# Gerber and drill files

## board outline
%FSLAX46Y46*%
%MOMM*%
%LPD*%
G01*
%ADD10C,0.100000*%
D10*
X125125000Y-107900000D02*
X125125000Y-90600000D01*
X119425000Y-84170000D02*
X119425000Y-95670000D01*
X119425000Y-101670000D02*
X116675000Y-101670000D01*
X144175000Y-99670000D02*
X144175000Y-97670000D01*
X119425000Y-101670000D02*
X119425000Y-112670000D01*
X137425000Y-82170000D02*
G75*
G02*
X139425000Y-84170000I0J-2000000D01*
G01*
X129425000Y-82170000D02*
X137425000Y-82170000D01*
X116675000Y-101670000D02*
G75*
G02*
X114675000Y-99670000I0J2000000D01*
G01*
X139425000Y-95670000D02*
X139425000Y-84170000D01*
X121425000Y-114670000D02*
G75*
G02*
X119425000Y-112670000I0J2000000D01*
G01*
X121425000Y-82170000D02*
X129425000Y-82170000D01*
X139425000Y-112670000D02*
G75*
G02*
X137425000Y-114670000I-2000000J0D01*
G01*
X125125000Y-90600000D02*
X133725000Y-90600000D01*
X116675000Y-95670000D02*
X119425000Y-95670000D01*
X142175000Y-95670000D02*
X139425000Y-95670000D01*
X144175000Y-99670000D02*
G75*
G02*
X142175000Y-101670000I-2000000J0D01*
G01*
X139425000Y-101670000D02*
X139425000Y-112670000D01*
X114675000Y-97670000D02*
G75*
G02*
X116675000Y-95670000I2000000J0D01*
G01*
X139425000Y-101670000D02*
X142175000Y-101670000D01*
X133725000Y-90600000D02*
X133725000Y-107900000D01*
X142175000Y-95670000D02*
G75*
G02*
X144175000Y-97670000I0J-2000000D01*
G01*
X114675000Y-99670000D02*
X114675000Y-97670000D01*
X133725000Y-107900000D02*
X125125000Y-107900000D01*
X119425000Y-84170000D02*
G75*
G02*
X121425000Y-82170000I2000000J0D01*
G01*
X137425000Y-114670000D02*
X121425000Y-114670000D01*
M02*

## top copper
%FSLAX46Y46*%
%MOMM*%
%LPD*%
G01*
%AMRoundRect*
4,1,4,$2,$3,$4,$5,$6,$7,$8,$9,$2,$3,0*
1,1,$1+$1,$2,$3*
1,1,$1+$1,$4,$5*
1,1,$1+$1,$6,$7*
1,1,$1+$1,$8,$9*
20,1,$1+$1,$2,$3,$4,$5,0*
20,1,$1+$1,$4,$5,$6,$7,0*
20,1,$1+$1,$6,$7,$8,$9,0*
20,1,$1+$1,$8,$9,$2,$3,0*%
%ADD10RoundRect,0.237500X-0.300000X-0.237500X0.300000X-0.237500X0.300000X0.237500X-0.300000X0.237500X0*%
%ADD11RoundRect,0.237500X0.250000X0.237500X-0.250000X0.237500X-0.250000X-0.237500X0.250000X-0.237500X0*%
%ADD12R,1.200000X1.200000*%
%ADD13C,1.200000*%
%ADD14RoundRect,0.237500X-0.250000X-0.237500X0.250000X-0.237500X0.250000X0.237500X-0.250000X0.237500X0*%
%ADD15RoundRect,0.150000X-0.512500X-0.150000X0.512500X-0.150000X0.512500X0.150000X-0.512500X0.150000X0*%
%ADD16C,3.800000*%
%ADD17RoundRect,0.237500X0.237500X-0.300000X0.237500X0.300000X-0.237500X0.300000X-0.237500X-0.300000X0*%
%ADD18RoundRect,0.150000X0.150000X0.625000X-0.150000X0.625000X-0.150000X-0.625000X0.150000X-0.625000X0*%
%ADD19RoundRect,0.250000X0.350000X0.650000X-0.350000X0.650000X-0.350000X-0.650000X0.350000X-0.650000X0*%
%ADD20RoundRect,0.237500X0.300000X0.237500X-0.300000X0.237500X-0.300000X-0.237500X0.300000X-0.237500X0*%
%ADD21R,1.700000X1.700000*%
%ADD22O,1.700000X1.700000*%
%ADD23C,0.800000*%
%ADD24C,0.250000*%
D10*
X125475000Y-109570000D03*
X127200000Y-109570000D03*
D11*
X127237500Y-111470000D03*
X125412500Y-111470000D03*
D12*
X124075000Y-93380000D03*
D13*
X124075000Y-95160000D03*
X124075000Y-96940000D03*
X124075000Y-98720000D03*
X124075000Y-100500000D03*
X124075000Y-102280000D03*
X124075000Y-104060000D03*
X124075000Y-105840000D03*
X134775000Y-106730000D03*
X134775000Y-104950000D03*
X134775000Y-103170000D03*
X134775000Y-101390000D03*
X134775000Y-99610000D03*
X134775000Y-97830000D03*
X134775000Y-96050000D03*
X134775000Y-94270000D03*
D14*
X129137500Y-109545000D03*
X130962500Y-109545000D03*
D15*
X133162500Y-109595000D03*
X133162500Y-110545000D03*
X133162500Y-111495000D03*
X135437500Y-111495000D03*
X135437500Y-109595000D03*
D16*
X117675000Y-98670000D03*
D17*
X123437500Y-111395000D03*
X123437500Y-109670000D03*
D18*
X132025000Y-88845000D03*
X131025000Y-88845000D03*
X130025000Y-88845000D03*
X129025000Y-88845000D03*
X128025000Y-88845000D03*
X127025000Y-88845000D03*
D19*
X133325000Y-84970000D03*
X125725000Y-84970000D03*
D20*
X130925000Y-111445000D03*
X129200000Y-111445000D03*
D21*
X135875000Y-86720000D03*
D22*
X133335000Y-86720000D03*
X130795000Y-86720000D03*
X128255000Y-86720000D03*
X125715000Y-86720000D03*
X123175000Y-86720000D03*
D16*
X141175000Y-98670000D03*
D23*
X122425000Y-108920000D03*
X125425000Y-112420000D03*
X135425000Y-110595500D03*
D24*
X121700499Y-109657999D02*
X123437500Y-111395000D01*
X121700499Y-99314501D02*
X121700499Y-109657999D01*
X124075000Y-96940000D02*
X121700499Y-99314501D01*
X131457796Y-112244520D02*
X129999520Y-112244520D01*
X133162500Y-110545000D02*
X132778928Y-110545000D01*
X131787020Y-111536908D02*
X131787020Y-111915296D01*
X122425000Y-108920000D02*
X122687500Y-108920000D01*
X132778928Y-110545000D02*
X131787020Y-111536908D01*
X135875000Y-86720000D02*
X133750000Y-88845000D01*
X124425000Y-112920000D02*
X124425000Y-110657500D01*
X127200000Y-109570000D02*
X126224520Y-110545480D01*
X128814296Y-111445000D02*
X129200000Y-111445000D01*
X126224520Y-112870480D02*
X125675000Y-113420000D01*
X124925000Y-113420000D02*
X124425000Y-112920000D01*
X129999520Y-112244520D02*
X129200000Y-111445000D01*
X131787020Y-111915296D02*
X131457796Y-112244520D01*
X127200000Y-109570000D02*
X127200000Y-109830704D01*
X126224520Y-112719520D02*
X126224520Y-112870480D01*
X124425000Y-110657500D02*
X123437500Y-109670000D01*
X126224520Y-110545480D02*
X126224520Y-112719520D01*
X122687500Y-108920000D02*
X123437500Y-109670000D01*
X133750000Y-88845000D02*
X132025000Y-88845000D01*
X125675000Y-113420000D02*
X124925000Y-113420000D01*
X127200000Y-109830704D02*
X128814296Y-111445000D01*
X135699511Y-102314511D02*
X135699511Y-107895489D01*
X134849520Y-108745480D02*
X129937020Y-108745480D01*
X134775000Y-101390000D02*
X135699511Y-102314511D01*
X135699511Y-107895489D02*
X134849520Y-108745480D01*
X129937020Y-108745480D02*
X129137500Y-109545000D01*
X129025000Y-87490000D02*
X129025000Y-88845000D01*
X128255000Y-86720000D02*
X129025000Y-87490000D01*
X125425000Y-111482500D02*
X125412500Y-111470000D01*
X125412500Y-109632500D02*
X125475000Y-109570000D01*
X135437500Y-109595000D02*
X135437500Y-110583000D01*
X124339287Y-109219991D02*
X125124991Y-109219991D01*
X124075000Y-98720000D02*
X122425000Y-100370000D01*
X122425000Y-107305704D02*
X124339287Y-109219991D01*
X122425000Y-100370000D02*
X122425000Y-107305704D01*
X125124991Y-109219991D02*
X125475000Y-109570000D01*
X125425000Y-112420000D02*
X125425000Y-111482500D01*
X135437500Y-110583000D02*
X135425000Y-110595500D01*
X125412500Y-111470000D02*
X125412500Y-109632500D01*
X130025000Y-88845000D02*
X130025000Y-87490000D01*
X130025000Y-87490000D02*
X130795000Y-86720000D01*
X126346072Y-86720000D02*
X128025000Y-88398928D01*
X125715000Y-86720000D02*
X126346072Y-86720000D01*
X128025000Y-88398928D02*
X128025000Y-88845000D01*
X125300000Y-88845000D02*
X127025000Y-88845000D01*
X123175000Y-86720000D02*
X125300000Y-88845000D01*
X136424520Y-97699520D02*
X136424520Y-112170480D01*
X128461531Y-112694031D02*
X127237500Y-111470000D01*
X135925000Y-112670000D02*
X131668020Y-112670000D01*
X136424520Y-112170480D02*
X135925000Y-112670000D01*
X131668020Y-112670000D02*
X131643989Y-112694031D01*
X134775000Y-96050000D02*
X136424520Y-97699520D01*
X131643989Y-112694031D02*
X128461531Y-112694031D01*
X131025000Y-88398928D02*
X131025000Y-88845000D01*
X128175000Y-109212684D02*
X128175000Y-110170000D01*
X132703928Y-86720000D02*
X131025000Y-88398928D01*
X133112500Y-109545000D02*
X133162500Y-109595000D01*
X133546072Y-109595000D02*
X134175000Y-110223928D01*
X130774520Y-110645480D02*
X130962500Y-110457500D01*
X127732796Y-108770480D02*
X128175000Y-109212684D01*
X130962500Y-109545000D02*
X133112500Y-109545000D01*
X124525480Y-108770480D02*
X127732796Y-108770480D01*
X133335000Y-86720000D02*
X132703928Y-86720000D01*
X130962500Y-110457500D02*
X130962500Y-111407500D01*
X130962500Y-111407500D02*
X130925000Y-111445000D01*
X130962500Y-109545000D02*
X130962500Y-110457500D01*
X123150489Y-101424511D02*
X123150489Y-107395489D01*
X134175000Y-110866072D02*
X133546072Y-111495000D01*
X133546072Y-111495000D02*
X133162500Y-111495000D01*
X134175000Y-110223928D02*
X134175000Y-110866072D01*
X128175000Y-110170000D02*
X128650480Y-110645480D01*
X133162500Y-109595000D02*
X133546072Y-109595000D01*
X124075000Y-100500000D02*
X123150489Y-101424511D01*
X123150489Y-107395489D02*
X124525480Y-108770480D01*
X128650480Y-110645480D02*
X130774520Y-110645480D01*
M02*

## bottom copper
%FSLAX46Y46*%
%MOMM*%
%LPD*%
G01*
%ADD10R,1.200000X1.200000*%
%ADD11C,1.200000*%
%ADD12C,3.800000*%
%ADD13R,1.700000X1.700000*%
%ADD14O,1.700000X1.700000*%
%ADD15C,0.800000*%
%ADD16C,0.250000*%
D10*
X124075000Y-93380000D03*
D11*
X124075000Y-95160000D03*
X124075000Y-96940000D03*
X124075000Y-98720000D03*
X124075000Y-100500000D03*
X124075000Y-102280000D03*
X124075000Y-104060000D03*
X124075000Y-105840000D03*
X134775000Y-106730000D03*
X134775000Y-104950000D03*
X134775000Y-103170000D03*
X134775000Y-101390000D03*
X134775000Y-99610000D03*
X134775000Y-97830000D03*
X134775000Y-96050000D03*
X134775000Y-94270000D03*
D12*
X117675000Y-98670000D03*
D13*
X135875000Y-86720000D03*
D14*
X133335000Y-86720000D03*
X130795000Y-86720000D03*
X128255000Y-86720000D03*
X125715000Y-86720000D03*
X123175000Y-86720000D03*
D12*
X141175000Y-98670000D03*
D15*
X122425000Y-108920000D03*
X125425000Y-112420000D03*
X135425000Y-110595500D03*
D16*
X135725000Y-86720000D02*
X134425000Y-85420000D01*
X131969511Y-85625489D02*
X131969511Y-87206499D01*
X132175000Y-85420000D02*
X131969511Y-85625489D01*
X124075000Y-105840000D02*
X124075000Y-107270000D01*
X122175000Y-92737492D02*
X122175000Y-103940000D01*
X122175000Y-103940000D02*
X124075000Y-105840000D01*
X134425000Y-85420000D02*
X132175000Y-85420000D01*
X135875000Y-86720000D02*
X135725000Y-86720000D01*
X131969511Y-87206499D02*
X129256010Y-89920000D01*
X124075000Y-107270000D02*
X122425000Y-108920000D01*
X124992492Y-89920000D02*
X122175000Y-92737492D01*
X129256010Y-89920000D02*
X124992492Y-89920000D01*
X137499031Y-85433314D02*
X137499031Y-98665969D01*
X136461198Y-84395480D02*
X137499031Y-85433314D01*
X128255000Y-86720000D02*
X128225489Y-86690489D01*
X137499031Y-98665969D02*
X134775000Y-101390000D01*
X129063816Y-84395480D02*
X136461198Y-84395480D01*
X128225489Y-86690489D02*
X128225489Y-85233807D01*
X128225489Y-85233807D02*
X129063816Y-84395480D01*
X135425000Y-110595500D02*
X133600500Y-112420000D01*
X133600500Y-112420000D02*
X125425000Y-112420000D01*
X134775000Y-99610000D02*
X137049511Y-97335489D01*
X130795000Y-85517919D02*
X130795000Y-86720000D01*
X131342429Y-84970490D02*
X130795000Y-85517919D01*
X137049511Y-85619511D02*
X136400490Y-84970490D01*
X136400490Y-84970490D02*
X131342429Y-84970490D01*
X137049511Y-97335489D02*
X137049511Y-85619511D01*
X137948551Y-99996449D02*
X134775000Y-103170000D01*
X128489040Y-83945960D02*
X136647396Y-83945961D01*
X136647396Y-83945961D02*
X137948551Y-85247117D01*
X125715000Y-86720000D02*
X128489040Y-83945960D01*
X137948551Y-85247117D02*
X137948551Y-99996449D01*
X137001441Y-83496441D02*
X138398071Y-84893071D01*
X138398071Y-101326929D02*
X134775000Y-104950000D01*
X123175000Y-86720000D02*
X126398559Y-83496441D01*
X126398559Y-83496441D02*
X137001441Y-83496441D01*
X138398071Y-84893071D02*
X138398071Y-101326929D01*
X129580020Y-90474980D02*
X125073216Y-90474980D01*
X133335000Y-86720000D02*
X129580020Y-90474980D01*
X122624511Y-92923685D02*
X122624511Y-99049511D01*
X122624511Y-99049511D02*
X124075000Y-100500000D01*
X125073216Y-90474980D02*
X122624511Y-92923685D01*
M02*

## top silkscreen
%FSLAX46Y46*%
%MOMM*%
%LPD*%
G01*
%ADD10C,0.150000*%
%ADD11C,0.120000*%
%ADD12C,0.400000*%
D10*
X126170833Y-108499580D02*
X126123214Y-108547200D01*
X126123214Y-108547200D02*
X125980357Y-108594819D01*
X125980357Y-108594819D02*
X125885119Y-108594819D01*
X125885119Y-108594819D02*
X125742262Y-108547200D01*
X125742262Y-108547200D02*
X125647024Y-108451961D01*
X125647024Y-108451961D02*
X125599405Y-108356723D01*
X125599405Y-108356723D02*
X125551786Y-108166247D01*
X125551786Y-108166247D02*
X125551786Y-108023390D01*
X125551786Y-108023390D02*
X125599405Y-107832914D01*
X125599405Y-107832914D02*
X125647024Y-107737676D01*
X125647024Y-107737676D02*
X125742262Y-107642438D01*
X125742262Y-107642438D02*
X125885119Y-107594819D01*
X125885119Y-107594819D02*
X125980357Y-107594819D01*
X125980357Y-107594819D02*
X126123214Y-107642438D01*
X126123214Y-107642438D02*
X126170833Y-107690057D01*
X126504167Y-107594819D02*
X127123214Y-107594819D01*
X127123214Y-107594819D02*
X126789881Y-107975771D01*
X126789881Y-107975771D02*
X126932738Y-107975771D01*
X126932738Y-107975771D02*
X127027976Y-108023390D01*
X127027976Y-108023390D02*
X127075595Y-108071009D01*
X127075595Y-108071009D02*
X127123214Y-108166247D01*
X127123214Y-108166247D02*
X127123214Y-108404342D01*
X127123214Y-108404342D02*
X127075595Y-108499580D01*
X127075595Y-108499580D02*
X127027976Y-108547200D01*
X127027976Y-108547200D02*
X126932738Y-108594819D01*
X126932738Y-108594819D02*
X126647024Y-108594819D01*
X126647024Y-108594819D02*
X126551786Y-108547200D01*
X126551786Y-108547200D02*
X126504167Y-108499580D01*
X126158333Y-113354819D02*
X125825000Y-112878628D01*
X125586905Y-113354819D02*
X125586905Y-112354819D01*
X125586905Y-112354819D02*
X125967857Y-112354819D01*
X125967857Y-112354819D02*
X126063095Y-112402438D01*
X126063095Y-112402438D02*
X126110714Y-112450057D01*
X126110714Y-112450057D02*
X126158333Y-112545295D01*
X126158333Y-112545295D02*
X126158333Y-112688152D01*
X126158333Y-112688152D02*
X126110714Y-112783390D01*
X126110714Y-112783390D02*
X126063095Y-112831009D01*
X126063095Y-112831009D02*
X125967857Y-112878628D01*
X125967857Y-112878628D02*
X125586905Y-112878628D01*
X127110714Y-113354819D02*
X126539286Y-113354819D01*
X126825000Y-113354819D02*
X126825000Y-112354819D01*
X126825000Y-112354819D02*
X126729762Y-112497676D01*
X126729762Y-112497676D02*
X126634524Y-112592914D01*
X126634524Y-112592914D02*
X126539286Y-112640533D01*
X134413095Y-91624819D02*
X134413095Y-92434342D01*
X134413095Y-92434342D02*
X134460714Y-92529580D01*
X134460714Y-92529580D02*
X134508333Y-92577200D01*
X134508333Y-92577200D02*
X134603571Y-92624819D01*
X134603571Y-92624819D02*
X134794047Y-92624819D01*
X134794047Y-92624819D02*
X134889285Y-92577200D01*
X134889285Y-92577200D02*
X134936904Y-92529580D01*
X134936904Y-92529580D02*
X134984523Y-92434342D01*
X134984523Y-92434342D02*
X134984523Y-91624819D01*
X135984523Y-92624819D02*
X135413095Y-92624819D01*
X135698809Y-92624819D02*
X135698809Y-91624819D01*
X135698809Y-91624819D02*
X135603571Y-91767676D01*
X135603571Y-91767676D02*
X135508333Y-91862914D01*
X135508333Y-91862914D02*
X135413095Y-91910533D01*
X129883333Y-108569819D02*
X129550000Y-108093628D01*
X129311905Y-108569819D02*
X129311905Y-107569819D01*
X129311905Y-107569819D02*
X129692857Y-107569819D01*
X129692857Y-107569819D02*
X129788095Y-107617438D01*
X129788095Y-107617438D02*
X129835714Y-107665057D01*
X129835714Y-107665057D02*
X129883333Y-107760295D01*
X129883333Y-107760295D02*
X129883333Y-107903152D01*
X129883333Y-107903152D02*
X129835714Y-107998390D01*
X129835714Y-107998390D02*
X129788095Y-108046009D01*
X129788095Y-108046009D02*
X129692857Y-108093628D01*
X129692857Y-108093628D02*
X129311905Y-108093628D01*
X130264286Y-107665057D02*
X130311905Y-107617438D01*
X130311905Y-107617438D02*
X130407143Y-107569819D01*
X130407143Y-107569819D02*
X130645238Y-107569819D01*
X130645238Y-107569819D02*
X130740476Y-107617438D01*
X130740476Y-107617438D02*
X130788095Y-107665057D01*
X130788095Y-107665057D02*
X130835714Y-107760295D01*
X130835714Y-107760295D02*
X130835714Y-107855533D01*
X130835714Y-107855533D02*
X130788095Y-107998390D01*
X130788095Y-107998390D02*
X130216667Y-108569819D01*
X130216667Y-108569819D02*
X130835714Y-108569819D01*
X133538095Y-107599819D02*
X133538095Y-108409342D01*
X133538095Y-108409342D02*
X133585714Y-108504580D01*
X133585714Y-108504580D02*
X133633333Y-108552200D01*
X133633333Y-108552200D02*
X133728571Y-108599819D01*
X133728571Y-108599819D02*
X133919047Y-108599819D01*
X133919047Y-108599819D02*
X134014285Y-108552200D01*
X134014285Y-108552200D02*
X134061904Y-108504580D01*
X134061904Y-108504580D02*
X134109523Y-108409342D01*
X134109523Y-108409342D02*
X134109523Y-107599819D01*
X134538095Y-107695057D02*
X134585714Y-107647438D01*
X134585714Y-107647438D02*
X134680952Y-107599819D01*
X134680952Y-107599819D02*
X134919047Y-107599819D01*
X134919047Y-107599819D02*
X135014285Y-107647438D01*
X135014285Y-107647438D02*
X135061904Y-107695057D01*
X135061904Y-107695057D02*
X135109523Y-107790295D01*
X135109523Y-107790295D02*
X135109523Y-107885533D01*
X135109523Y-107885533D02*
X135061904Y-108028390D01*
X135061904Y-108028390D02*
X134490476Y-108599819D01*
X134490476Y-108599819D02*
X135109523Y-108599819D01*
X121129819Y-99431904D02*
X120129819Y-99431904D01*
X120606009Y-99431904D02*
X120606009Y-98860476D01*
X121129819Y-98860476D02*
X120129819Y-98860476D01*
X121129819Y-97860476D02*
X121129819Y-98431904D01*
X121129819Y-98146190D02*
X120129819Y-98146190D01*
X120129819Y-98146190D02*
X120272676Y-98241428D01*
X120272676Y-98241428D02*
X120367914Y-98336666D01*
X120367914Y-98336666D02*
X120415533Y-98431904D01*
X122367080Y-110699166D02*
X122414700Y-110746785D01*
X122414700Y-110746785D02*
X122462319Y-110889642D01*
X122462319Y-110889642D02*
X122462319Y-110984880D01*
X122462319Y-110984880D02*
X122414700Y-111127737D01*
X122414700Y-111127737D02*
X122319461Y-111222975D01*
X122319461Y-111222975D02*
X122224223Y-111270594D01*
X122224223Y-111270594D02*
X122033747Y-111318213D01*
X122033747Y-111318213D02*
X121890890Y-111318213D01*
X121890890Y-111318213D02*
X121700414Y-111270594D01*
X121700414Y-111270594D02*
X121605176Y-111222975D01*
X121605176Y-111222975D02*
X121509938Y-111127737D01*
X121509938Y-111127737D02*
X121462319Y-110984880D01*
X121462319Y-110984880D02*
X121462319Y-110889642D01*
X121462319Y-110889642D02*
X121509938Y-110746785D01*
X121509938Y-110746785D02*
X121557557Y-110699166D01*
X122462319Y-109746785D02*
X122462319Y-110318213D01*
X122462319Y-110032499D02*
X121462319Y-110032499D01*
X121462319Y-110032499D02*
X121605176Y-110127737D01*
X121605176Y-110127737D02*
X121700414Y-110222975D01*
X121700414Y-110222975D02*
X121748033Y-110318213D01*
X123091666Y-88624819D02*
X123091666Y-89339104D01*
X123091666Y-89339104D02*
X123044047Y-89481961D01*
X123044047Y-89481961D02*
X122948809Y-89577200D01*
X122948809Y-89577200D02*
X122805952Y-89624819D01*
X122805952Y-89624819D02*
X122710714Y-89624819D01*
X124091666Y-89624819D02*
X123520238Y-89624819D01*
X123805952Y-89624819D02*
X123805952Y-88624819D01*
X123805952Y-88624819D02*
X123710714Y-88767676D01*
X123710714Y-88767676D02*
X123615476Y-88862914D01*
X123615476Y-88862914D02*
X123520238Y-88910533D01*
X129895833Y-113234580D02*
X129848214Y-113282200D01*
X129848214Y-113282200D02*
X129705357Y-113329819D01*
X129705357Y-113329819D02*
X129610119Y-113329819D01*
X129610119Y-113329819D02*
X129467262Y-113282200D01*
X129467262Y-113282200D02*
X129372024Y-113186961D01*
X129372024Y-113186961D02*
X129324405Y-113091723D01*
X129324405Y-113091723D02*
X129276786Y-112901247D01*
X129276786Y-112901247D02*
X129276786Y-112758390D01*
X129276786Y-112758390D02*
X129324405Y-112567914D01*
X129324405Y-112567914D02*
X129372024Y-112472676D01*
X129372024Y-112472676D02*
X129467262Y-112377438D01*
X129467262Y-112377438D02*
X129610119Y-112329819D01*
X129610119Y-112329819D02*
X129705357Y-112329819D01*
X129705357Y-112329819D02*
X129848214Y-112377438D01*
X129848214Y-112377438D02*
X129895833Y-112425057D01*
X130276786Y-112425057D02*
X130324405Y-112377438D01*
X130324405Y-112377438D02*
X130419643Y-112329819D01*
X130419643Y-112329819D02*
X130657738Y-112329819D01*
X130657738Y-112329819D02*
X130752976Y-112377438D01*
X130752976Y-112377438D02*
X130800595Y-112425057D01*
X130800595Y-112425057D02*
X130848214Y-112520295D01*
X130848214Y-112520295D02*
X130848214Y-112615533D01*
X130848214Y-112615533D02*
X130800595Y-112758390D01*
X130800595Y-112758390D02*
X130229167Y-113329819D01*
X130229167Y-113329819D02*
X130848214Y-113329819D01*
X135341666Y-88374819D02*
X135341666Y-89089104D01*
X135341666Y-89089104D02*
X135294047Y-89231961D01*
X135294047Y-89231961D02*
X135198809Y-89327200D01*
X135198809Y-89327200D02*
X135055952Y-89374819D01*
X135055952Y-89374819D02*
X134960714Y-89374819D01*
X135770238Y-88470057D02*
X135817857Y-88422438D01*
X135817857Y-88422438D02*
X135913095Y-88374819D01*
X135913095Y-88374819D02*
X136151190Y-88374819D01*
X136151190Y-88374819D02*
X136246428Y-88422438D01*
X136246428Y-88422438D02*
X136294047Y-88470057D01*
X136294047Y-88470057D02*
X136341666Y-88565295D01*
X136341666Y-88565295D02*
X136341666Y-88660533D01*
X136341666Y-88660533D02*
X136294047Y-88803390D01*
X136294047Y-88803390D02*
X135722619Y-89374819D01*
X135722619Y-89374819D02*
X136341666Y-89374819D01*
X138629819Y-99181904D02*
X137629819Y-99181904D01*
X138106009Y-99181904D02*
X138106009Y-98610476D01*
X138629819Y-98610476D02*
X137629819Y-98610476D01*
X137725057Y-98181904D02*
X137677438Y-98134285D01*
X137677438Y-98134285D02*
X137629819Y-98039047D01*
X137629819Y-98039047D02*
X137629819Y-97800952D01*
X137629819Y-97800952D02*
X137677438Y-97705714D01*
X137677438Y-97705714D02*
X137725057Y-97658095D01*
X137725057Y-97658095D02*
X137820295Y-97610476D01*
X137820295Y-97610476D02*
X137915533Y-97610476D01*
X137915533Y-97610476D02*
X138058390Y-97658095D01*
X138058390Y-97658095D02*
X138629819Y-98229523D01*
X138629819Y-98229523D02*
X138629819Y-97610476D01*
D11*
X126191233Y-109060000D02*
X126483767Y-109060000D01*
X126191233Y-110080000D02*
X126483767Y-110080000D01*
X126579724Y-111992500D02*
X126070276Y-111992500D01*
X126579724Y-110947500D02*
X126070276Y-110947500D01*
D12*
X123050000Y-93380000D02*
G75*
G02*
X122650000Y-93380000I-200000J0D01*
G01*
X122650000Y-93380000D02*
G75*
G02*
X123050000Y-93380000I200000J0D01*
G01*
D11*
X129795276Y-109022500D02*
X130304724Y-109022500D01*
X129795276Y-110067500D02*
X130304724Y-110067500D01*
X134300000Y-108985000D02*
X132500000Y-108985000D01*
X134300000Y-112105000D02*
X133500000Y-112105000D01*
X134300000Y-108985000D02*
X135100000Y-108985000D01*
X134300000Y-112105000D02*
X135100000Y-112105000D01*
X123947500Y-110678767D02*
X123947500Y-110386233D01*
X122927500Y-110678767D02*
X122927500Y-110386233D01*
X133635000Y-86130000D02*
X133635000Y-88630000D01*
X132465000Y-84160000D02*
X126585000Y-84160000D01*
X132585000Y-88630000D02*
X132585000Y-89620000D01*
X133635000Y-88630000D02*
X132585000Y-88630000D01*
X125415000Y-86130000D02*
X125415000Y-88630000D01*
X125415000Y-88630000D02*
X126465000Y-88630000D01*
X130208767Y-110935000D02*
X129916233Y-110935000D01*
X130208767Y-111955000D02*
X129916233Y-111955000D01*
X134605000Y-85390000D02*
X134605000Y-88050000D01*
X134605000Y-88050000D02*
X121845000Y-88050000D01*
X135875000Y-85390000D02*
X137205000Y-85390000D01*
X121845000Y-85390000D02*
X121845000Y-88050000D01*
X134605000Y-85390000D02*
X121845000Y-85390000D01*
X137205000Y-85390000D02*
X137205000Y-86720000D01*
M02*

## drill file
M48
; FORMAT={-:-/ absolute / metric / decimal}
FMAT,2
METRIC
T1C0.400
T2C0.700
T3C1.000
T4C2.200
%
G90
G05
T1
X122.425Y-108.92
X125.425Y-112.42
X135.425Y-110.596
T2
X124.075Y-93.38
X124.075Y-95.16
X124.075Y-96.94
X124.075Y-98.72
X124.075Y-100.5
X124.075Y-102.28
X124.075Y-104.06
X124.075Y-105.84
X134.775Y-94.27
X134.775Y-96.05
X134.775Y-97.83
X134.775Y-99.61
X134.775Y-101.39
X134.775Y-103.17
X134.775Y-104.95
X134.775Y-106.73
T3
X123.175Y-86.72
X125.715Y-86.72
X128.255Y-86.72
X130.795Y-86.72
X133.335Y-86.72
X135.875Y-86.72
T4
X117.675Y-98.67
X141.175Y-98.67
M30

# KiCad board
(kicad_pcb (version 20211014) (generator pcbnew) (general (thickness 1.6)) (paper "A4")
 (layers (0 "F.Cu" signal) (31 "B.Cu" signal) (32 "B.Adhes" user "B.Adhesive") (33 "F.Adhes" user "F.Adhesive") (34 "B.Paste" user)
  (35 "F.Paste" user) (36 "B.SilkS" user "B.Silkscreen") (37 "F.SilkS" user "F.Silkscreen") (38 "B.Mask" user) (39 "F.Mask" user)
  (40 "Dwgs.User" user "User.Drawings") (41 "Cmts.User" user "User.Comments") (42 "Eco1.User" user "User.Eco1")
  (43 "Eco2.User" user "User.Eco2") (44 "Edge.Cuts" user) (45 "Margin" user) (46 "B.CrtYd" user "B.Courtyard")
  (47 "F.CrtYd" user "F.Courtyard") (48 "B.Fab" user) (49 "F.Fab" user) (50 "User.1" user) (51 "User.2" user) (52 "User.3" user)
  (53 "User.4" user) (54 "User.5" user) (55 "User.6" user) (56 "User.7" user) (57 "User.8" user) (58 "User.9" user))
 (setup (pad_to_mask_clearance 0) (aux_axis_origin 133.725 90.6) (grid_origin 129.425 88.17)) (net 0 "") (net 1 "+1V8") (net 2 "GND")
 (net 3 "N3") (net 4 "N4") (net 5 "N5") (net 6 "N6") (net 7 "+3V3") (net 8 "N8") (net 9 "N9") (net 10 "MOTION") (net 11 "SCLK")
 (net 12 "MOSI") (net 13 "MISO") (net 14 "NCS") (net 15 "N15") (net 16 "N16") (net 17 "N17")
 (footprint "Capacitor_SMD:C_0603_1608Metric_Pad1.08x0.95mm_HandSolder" (layer "F.Cu") (at 126.3375 109.57)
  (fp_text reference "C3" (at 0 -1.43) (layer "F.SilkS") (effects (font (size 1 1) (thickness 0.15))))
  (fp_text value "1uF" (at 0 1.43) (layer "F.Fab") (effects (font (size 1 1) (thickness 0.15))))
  (fp_line (start -0.146267 -0.51) (end 0.146267 -0.51) (layer "F.SilkS") (width 0.12))
  (fp_line (start -0.146267 0.51) (end 0.146267 0.51) (layer "F.SilkS") (width 0.12))
  (pad "1" smd roundrect (at -0.8625 0) (size 1.075 0.95) (layers "F.Cu" "F.Paste" "F.Mask") (roundrect_rratio 0.25) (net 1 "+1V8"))
  (pad "2" smd roundrect (at 0.8625 0) (size 1.075 0.95) (layers "F.Cu" "F.Paste" "F.Mask") (roundrect_rratio 0.25) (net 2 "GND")))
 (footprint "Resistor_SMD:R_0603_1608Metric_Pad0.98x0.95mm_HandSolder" (layer "F.Cu") (at 126.325 111.47 180)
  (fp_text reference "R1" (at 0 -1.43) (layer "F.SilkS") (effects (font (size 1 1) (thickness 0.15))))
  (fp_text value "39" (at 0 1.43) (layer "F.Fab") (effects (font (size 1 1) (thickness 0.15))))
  (fp_line (start -0.254724 -0.5225) (end 0.254724 -0.5225) (layer "F.SilkS") (width 0.12))
  (fp_line (start -0.254724 0.5225) (end 0.254724 0.5225) (layer "F.SilkS") (width 0.12))
  (pad "1" smd roundrect (at -0.9125 0 180) (size 0.975 0.95) (layers "F.Cu" "F.Paste" "F.Mask") (roundrect_rratio 0.25) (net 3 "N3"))
  (pad "2" smd roundrect (at 0.9125 0 180) (size 0.975 0.95) (layers "F.Cu" "F.Paste" "F.Mask") (roundrect_rratio 0.25) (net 1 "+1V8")))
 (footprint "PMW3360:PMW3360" (layer "F.Cu") (at 124.075 93.38)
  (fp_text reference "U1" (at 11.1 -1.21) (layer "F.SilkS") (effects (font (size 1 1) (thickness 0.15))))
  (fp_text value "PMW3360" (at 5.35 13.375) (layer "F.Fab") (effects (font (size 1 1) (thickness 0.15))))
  (fp_circle (center -1.225 0) (end -1.025 0) (layer "F.SilkS") (width 0.4) (fill none))
  (pad "1" thru_hole rect (at 0 0) (size 1.2 1.2) (drill 0.7) (layers *.Cu *.Mask) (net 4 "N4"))
  (pad "2" thru_hole circle (at 0 1.78) (size 1.2 1.2) (drill 0.7) (layers *.Cu *.Mask) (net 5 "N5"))
  (pad "3" thru_hole circle (at 0 3.56) (size 1.2 1.2) (drill 0.7) (layers *.Cu *.Mask) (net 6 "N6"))
  (pad "4" thru_hole circle (at 0 5.34) (size 1.2 1.2) (drill 0.7) (layers *.Cu *.Mask) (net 1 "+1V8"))
  (pad "5" thru_hole circle (at 0 7.12) (size 1.2 1.2) (drill 0.7) (layers *.Cu *.Mask) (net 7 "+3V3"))
  (pad "6" thru_hole circle (at 0 8.9) (size 1.2 1.2) (drill 0.7) (layers *.Cu *.Mask) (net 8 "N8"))
  (pad "7" thru_hole circle (at 0 10.68) (size 1.2 1.2) (drill 0.7) (layers *.Cu *.Mask) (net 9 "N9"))
  (pad "8" thru_hole circle (at 0 12.46) (size 1.2 1.2) (drill 0.7) (layers *.Cu *.Mask) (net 2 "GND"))
  (pad "9" thru_hole circle (at 10.7 13.35) (size 1.2 1.2) (drill 0.7) (layers *.Cu *.Mask) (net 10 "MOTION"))
  (pad "10" thru_hole circle (at 10.7 11.57) (size 1.2 1.2) (drill 0.7) (layers *.Cu *.Mask) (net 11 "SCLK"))
  (pad "11" thru_hole circle (at 10.7 9.79) (size 1.2 1.2) (drill 0.7) (layers *.Cu *.Mask) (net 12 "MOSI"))
  (pad "12" thru_hole circle (at 10.7 8.01) (size 1.2 1.2) (drill 0.7) (layers *.Cu *.Mask) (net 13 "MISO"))
  (pad "13" thru_hole circle (at 10.7 6.23) (size 1.2 1.2) (drill 0.7) (layers *.Cu *.Mask) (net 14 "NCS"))
  (pad "14" thru_hole circle (at 10.7 4.45) (size 1.2 1.2) (drill 0.7) (layers *.Cu *.Mask) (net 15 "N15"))
  (pad "15" thru_hole circle (at 10.7 2.67) (size 1.2 1.2) (drill 0.7) (layers *.Cu *.Mask) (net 3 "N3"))
  (pad "16" thru_hole circle (at 10.7 0.89) (size 1.2 1.2) (drill 0.7) (layers *.Cu *.Mask) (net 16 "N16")))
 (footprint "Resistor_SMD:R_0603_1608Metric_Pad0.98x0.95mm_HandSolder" (layer "F.Cu") (at 130.05 109.545)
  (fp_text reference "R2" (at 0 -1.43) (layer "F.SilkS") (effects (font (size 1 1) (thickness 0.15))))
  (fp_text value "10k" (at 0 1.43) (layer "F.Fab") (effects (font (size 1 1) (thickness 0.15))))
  (fp_line (start -0.254724 -0.5225) (end 0.254724 -0.5225) (layer "F.SilkS") (width 0.12))
  (fp_line (start -0.254724 0.5225) (end 0.254724 0.5225) (layer "F.SilkS") (width 0.12))
  (pad "1" smd roundrect (at -0.9125 0) (size 0.975 0.95) (layers "F.Cu" "F.Paste" "F.Mask") (roundrect_rratio 0.25) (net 13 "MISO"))
  (pad "2" smd roundrect (at 0.9125 0) (size 0.975 0.95) (layers "F.Cu" "F.Paste" "F.Mask") (roundrect_rratio 0.25) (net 7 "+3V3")))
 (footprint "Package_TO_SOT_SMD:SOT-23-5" (layer "F.Cu") (at 134.3 110.545)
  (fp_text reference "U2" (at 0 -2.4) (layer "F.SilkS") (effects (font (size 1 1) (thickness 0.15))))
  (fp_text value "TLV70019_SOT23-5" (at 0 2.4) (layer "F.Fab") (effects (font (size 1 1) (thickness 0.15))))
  (fp_line (start 0 -1.56) (end -1.8 -1.56) (layer "F.SilkS") (width 0.12))
  (fp_line (start 0 1.56) (end -0.8 1.56) (layer "F.SilkS") (width 0.12))
  (fp_line (start 0 -1.56) (end 0.8 -1.56) (layer "F.SilkS") (width 0.12))
  (fp_line (start 0 1.56) (end 0.8 1.56) (layer "F.SilkS") (width 0.12))
  (pad "1" smd roundrect (at -1.1375 -0.95) (size 1.325 0.6) (layers "F.Cu" "F.Paste" "F.Mask") (roundrect_rratio 0.25) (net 7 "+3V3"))
  (pad "2" smd roundrect (at -1.1375 0) (size 1.325 0.6) (layers "F.Cu" "F.Paste" "F.Mask") (roundrect_rratio 0.25) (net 2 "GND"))
  (pad "3" smd roundrect (at -1.1375 0.95) (size 1.325 0.6) (layers "F.Cu" "F.Paste" "F.Mask") (roundrect_rratio 0.25) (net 7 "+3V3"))
  (pad "4" smd roundrect (at 1.1375 0.95) (size 1.325 0.6) (layers "F.Cu" "F.Paste" "F.Mask") (roundrect_rratio 0.25) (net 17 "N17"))
  (pad "5" smd roundrect (at 1.1375 -0.95) (size 1.325 0.6) (layers "F.Cu" "F.Paste" "F.Mask") (roundrect_rratio 0.25) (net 1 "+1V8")))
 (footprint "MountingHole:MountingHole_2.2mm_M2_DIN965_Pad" (layer "F.Cu") (at 117.675 98.67)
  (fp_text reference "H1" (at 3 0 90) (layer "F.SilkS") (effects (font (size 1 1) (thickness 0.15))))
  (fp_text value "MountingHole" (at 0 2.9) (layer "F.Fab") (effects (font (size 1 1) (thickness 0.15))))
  (pad "1" thru_hole circle (at 0 0) (size 3.8 3.8) (drill 2.2) (layers *.Cu *.Mask)))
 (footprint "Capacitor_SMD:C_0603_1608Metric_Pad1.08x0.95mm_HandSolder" (layer "F.Cu") (at 123.4375 110.5325 90)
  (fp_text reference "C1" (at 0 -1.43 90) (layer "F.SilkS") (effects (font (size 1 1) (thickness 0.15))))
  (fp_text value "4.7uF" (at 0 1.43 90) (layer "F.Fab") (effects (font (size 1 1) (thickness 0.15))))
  (fp_line (start -0.146267 0.51) (end 0.146267 0.51) (layer "F.SilkS") (width 0.12))
  (fp_line (start -0.146267 -0.51) (end 0.146267 -0.51) (layer "F.SilkS") (width 0.12))
  (pad "1" smd roundrect (at -0.8625 0 90) (size 1.075 0.95) (layers "F.Cu" "F.Paste" "F.Mask") (roundrect_rratio 0.25) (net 6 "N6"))
  (pad "2" smd roundrect (at 0.8625 0 90) (size 1.075 0.95) (layers "F.Cu" "F.Paste" "F.Mask") (roundrect_rratio 0.25) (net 2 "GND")))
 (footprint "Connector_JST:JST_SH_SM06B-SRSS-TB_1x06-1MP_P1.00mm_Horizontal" (layer "F.Cu") (at 129.525 86.845 180)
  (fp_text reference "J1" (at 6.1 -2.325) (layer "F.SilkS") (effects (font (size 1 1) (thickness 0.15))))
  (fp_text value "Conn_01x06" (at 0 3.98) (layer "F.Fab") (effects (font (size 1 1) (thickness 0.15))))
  (fp_line (start -4.11 0.715) (end -4.11 -1.785) (layer "F.SilkS") (width 0.12))
  (fp_line (start -2.94 2.685) (end 2.94 2.685) (layer "F.SilkS") (width 0.12))
  (fp_line (start -3.06 -1.785) (end -3.06 -2.775) (layer "F.SilkS") (width 0.12))
  (fp_line (start -4.11 -1.785) (end -3.06 -1.785) (layer "F.SilkS") (width 0.12))
  (fp_line (start 4.11 0.715) (end 4.11 -1.785) (layer "F.SilkS") (width 0.12))
  (fp_line (start 4.11 -1.785) (end 3.06 -1.785) (layer "F.SilkS") (width 0.12))
  (pad "1" smd roundrect (at -2.5 -2 180) (size 0.6 1.55) (layers "F.Cu" "F.Paste" "F.Mask") (roundrect_rratio 0.25) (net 2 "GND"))
  (pad "2" smd roundrect (at -1.5 -2 180) (size 0.6 1.55) (layers "F.Cu" "F.Paste" "F.Mask") (roundrect_rratio 0.25) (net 7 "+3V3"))
  (pad "3" smd roundrect (at -0.5 -2 180) (size 0.6 1.55) (layers "F.Cu" "F.Paste" "F.Mask") (roundrect_rratio 0.25) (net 14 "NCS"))
  (pad "4" smd roundrect (at 0.5 -2 180) (size 0.6 1.55) (layers "F.Cu" "F.Paste" "F.Mask") (roundrect_rratio 0.25) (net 13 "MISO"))
  (pad "5" smd roundrect (at 1.5 -2 180) (size 0.6 1.55) (layers "F.Cu" "F.Paste" "F.Mask") (roundrect_rratio 0.25) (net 12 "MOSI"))
  (pad "6" smd roundrect (at 2.5 -2 180) (size 0.6 1.55) (layers "F.Cu" "F.Paste" "F.Mask") (roundrect_rratio 0.25) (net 11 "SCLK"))
  (pad "MP" smd roundrect (at -3.8 1.875 180) (size 1.2 1.8) (layers "F.Cu" "F.Paste" "F.Mask") (roundrect_rratio 0.208333))
  (pad "MP" smd roundrect (at 3.8 1.875 180) (size 1.2 1.8) (layers "F.Cu" "F.Paste" "F.Mask") (roundrect_rratio 0.208333)))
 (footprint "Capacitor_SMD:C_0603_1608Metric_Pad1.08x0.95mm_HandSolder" (layer "F.Cu") (at 130.0625 111.445 180)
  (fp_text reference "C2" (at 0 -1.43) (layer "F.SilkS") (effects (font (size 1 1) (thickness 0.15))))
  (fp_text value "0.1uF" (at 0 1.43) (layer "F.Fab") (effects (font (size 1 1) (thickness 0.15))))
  (fp_line (start -0.146267 0.51) (end 0.146267 0.51) (layer "F.SilkS") (width 0.12))
  (fp_line (start -0.146267 -0.51) (end 0.146267 -0.51) (layer "F.SilkS") (width 0.12))
  (pad "1" smd roundrect (at -0.8625 0 180) (size 1.075 0.95) (layers "F.Cu" "F.Paste" "F.Mask") (roundrect_rratio 0.25) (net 7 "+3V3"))
  (pad "2" smd roundrect (at 0.8625 0 180) (size 1.075 0.95) (layers "F.Cu" "F.Paste" "F.Mask") (roundrect_rratio 0.25) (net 2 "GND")))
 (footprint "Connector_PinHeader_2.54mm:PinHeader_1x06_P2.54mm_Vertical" (layer "F.Cu") (at 135.875 86.72 -90)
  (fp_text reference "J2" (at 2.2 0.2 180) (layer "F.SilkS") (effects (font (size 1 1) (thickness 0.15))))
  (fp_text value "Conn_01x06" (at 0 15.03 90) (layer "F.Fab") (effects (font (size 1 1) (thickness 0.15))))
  (fp_line (start -1.33 1.27) (end 1.33 1.27) (layer "F.SilkS") (width 0.12))
  (fp_line (start 1.33 1.27) (end 1.33 14.03) (layer "F.SilkS") (width 0.12))
  (fp_line (start -1.33 0) (end -1.33 -1.33) (layer "F.SilkS") (width 0.12))
  (fp_line (start -1.33 14.03) (end 1.33 14.03) (layer "F.SilkS") (width 0.12))
  (fp_line (start -1.33 1.27) (end -1.33 14.03) (layer "F.SilkS") (width 0.12))
  (fp_line (start -1.33 -1.33) (end 0 -1.33) (layer "F.SilkS") (width 0.12))
  (pad "1" thru_hole rect (at 0 0 270) (size 1.7 1.7) (drill 1) (layers *.Cu *.Mask) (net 2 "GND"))
  (pad "2" thru_hole oval (at 0 2.54 270) (size 1.7 1.7) (drill 1) (layers *.Cu *.Mask) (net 7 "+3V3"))
  (pad "3" thru_hole oval (at 0 5.08 270) (size 1.7 1.7) (drill 1) (layers *.Cu *.Mask) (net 14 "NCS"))
  (pad "4" thru_hole oval (at 0 7.62 270) (size 1.7 1.7) (drill 1) (layers *.Cu *.Mask) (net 13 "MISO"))
  (pad "5" thru_hole oval (at 0 10.16 270) (size 1.7 1.7) (drill 1) (layers *.Cu *.Mask) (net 12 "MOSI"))
  (pad "6" thru_hole oval (at 0 12.7 270) (size 1.7 1.7) (drill 1) (layers *.Cu *.Mask) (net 11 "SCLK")))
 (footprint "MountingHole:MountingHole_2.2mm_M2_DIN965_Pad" (layer "F.Cu") (at 141.175 98.67)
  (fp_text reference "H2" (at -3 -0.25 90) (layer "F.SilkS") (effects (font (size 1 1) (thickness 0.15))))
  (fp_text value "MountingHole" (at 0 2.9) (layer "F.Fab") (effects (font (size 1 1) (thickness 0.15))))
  (pad "1" thru_hole circle (at 0 0) (size 3.8 3.8) (drill 2.2) (layers *.Cu *.Mask)))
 (gr_line (start 125.125 107.9) (end 125.125 90.6) (layer "Edge.Cuts") (width 0.1))
 (gr_line (start 119.425 84.17) (end 119.425 95.67) (layer "Edge.Cuts") (width 0.1))
 (gr_line (start 119.425 101.67) (end 116.675 101.67) (layer "Edge.Cuts") (width 0.1))
 (gr_line (start 144.175 99.67) (end 144.175 97.67) (layer "Edge.Cuts") (width 0.1))
 (gr_line (start 119.425 101.67) (end 119.425 112.67) (layer "Edge.Cuts") (width 0.1))
 (gr_arc (start 137.425 82.17) (mid 138.839214 82.755786) (end 139.425 84.17) (layer "Edge.Cuts") (width 0.1))
 (gr_line (start 129.425 82.17) (end 137.425 82.17) (layer "Edge.Cuts") (width 0.1))
 (gr_arc (start 116.675 101.67) (mid 115.260786 101.084214) (end 114.675 99.67) (layer "Edge.Cuts") (width 0.1))
 (gr_line (start 139.425 95.67) (end 139.425 84.17) (layer "Edge.Cuts") (width 0.1))
 (gr_arc (start 121.425 114.67) (mid 120.010786 114.084214) (end 119.425 112.67) (layer "Edge.Cuts") (width 0.1))
 (gr_line (start 121.425 82.17) (end 129.425 82.17) (layer "Edge.Cuts") (width 0.1))
 (gr_arc (start 139.425 112.67) (mid 138.839214 114.084214) (end 137.425 114.67) (layer "Edge.Cuts") (width 0.1))
 (gr_line (start 125.125 90.6) (end 133.725 90.6) (layer "Edge.Cuts") (width 0.1))
 (gr_line (start 116.675 95.67) (end 119.425 95.67) (layer "Edge.Cuts") (width 0.1))
 (gr_line (start 142.175 95.67) (end 139.425 95.67) (layer "Edge.Cuts") (width 0.1))
 (gr_arc (start 144.175 99.67) (mid 143.589214 101.084214) (end 142.175 101.67) (layer "Edge.Cuts") (width 0.1))
 (gr_line (start 139.425 101.67) (end 139.425 112.67) (layer "Edge.Cuts") (width 0.1))
 (gr_arc (start 114.675 97.67) (mid 115.260786 96.255786) (end 116.675 95.67) (layer "Edge.Cuts") (width 0.1))
 (gr_line (start 139.425 101.67) (end 142.175 101.67) (layer "Edge.Cuts") (width 0.1))
 (gr_line (start 133.725 90.6) (end 133.725 107.9) (layer "Edge.Cuts") (width 0.1))
 (gr_arc (start 142.175 95.67) (mid 143.589214 96.255786) (end 144.175 97.67) (layer "Edge.Cuts") (width 0.1))
 (gr_line (start 114.675 99.67) (end 114.675 97.67) (layer "Edge.Cuts") (width 0.1))
 (gr_line (start 133.725 107.9) (end 125.125 107.9) (layer "Edge.Cuts") (width 0.1))
 (gr_arc (start 119.425 84.17) (mid 120.010786 82.755786) (end 121.425 82.17) (layer "Edge.Cuts") (width 0.1))
 (gr_line (start 137.425 114.67) (end 121.425 114.67) (layer "Edge.Cuts") (width 0.1))
 (segment (start 121.700499 109.657999) (end 123.4375 111.395) (width 0.25) (layer "F.Cu") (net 6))
 (segment (start 121.700499 99.314501) (end 121.700499 109.657999) (width 0.25) (layer "F.Cu") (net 6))
 (segment (start 124.075 96.94) (end 121.700499 99.314501) (width 0.25) (layer "F.Cu") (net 6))
 (segment (start 131.457796 112.24452) (end 129.99952 112.24452) (width 0.25) (layer "F.Cu") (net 2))
 (segment (start 133.1625 110.545) (end 132.778928 110.545) (width 0.25) (layer "F.Cu") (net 2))
 (segment (start 131.78702 111.536908) (end 131.78702 111.915296) (width 0.25) (layer "F.Cu") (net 2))
 (segment (start 122.425 108.92) (end 122.6875 108.92) (width 0.25) (layer "F.Cu") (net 2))
 (segment (start 132.778928 110.545) (end 131.78702 111.536908) (width 0.25) (layer "F.Cu") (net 2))
 (segment (start 135.875 86.72) (end 133.75 88.845) (width 0.25) (layer "F.Cu") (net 2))
 (segment (start 124.425 112.92) (end 124.425 110.6575) (width 0.25) (layer "F.Cu") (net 2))
 (segment (start 127.2 109.57) (end 126.22452 110.54548) (width 0.25) (layer "F.Cu") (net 2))
 (segment (start 128.814296 111.445) (end 129.2 111.445) (width 0.25) (layer "F.Cu") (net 2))
 (segment (start 126.22452 112.87048) (end 125.675 113.42) (width 0.25) (layer "F.Cu") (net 2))
 (segment (start 124.925 113.42) (end 124.425 112.92) (width 0.25) (layer "F.Cu") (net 2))
 (segment (start 129.99952 112.24452) (end 129.2 111.445) (width 0.25) (layer "F.Cu") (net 2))
 (segment (start 131.78702 111.915296) (end 131.457796 112.24452) (width 0.25) (layer "F.Cu") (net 2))
 (segment (start 127.2 109.57) (end 127.2 109.830704) (width 0.25) (layer "F.Cu") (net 2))
 (segment (start 126.22452 112.71952) (end 126.22452 112.87048) (width 0.25) (layer "F.Cu") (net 2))
 (segment (start 124.425 110.6575) (end 123.4375 109.67) (width 0.25) (layer "F.Cu") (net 2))
 (segment (start 126.22452 110.54548) (end 126.22452 112.71952) (width 0.25) (layer "F.Cu") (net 2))
 (segment (start 122.6875 108.92) (end 123.4375 109.67) (width 0.25) (layer "F.Cu") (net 2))
 (segment (start 133.75 88.845) (end 132.025 88.845) (width 0.25) (layer "F.Cu") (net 2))
 (segment (start 125.675 113.42) (end 124.925 113.42) (width 0.25) (layer "F.Cu") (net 2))
 (segment (start 127.2 109.830704) (end 128.814296 111.445) (width 0.25) (layer "F.Cu") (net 2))
 (via (at 122.425 108.92) (size 0.8) (drill 0.4) (layers "F.Cu" "B.Cu") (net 2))
 (segment (start 135.725 86.72) (end 134.425 85.42) (width 0.25) (layer "B.Cu") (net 2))
 (segment (start 131.969511 85.625489) (end 131.969511 87.206499) (width 0.25) (layer "B.Cu") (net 2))
 (segment (start 132.175 85.42) (end 131.969511 85.625489) (width 0.25) (layer "B.Cu") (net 2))
 (segment (start 124.075 105.84) (end 124.075 107.27) (width 0.25) (layer "B.Cu") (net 2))
 (segment (start 122.175 92.737492) (end 122.175 103.94) (width 0.25) (layer "B.Cu") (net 2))
 (segment (start 122.175 103.94) (end 124.075 105.84) (width 0.25) (layer "B.Cu") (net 2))
 (segment (start 134.425 85.42) (end 132.175 85.42) (width 0.25) (layer "B.Cu") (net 2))
 (segment (start 135.875 86.72) (end 135.725 86.72) (width 0.25) (layer "B.Cu") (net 2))
 (segment (start 131.969511 87.206499) (end 129.25601 89.92) (width 0.25) (layer "B.Cu") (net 2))
 (segment (start 124.075 107.27) (end 122.425 108.92) (width 0.25) (layer "B.Cu") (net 2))
 (segment (start 124.992492 89.92) (end 122.175 92.737492) (width 0.25) (layer "B.Cu") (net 2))
 (segment (start 129.25601 89.92) (end 124.992492 89.92) (width 0.25) (layer "B.Cu") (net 2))
 (segment (start 135.699511 102.314511) (end 135.699511 107.895489) (width 0.25) (layer "F.Cu") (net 13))
 (segment (start 134.84952 108.74548) (end 129.93702 108.74548) (width 0.25) (layer "F.Cu") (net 13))
 (segment (start 134.775 101.39) (end 135.699511 102.314511) (width 0.25) (layer "F.Cu") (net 13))
 (segment (start 135.699511 107.895489) (end 134.84952 108.74548) (width 0.25) (layer "F.Cu") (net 13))
 (segment (start 129.93702 108.74548) (end 129.1375 109.545) (width 0.25) (layer "F.Cu") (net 13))
 (segment (start 129.025 87.49) (end 129.025 88.845) (width 0.25) (layer "F.Cu") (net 13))
 (segment (start 128.255 86.72) (end 129.025 87.49) (width 0.25) (layer "F.Cu") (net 13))
 (segment (start 137.499031 85.433314) (end 137.499031 98.665969) (width 0.25) (layer "B.Cu") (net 13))
 (segment (start 136.461198 84.39548) (end 137.499031 85.433314) (width 0.25) (layer "B.Cu") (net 13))
 (segment (start 128.255 86.72) (end 128.225489 86.690489) (width 0.25) (layer "B.Cu") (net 13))
 (segment (start 137.499031 98.665969) (end 134.775 101.39) (width 0.25) (layer "B.Cu") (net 13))
 (segment (start 129.063816 84.39548) (end 136.461198 84.39548) (width 0.25) (layer "B.Cu") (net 13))
 (segment (start 128.225489 86.690489) (end 128.225489 85.233807) (width 0.25) (layer "B.Cu") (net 13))
 (segment (start 128.225489 85.233807) (end 129.063816 84.39548) (width 0.25) (layer "B.Cu") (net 13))
 (segment (start 125.425 111.4825) (end 125.4125 111.47) (width 0.25) (layer "F.Cu") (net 1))
 (segment (start 125.4125 109.6325) (end 125.475 109.57) (width 0.25) (layer "F.Cu") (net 1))
 (segment (start 135.4375 109.595) (end 135.4375 110.583) (width 0.25) (layer "F.Cu") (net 1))
 (segment (start 124.339287 109.219991) (end 125.124991 109.219991) (width 0.25) (layer "F.Cu") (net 1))
 (segment (start 124.075 98.72) (end 122.425 100.37) (width 0.25) (layer "F.Cu") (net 1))
 (segment (start 122.425 107.305704) (end 124.339287 109.219991) (width 0.25) (layer "F.Cu") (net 1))
 (segment (start 122.425 100.37) (end 122.425 107.305704) (width 0.25) (layer "F.Cu") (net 1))
 (segment (start 125.124991 109.219991) (end 125.475 109.57) (width 0.25) (layer "F.Cu") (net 1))
 (segment (start 125.425 112.42) (end 125.425 111.4825) (width 0.25) (layer "F.Cu") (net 1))
 (segment (start 135.4375 110.583) (end 135.425 110.5955) (width 0.25) (layer "F.Cu") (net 1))
 (segment (start 125.4125 111.47) (end 125.4125 109.6325) (width 0.25) (layer "F.Cu") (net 1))
 (via (at 125.425 112.42) (size 0.8) (drill 0.4) (layers "F.Cu" "B.Cu") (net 1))
 (via (at 135.425 110.5955) (size 0.8) (drill 0.4) (layers "F.Cu" "B.Cu") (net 1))
 (segment (start 135.425 110.5955) (end 133.6005 112.42) (width 0.25) (layer "B.Cu") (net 1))
 (segment (start 133.6005 112.42) (end 125.425 112.42) (width 0.25) (layer "B.Cu") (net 1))
 (segment (start 130.025 88.845) (end 130.025 87.49) (width 0.25) (layer "F.Cu") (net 14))
 (segment (start 130.025 87.49) (end 130.795 86.72) (width 0.25) (layer "F.Cu") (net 14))
 (segment (start 134.775 99.61) (end 137.049511 97.335489) (width 0.25) (layer "B.Cu") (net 14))
 (segment (start 130.795 85.517919) (end 130.795 86.72) (width 0.25) (layer "B.Cu") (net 14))
 (segment (start 131.342429 84.97049) (end 130.795 85.517919) (width 0.25) (layer "B.Cu") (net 14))
 (segment (start 137.049511 85.619511) (end 136.40049 84.97049) (width 0.25) (layer "B.Cu") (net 14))
 (segment (start 136.40049 84.97049) (end 131.342429 84.97049) (width 0.25) (layer "B.Cu") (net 14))
 (segment (start 137.049511 97.335489) (end 137.049511 85.619511) (width 0.25) (layer "B.Cu") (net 14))
 (segment (start 126.346072 86.72) (end 128.025 88.398928) (width 0.25) (layer "F.Cu") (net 12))
 (segment (start 125.715 86.72) (end 126.346072 86.72) (width 0.25) (layer "F.Cu") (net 12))
 (segment (start 128.025 88.398928) (end 128.025 88.845) (width 0.25) (layer "F.Cu") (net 12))
 (segment (start 137.948551 99.996449) (end 134.775 103.17) (width 0.25) (layer "B.Cu") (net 12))
 (segment (start 128.48904 83.94596) (end 136.647396 83.945961) (width 0.25) (layer "B.Cu") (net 12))
 (segment (start 136.647396 83.945961) (end 137.948551 85.247117) (width 0.25) (layer "B.Cu") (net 12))
 (segment (start 125.715 86.72) (end 128.48904 83.94596) (width 0.25) (layer "B.Cu") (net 12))
 (segment (start 137.948551 85.247117) (end 137.948551 99.996449) (width 0.25) (layer "B.Cu") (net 12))
 (segment (start 125.3 88.845) (end 127.025 88.845) (width 0.25) (layer "F.Cu") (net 11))
 (segment (start 123.175 86.72) (end 125.3 88.845) (width 0.25) (layer "F.Cu") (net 11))
 (segment (start 137.001441 83.496441) (end 138.398071 84.893071) (width 0.25) (layer "B.Cu") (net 11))
 (segment (start 138.398071 101.326929) (end 134.775 104.95) (width 0.25) (layer "B.Cu") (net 11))
 (segment (start 123.175 86.72) (end 126.398559 83.496441) (width 0.25) (layer "B.Cu") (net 11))
 (segment (start 126.398559 83.496441) (end 137.001441 83.496441) (width 0.25) (layer "B.Cu") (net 11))
 (segment (start 138.398071 84.893071) (end 138.398071 101.326929) (width 0.25) (layer "B.Cu") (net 11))
 (segment (start 136.42452 97.69952) (end 136.42452 112.17048) (width 0.25) (layer "F.Cu") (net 3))
 (segment (start 128.461531 112.694031) (end 127.2375 111.47) (width 0.25) (layer "F.Cu") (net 3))
 (segment (start 135.925 112.67) (end 131.66802 112.67) (width 0.25) (layer "F.Cu") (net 3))
 (segment (start 136.42452 112.17048) (end 135.925 112.67) (width 0.25) (layer "F.Cu") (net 3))
 (segment (start 131.66802 112.67) (end 131.643989 112.694031) (width 0.25) (layer "F.Cu") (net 3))
 (segment (start 134.775 96.05) (end 136.42452 97.69952) (width 0.25) (layer "F.Cu") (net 3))
 (segment (start 131.643989 112.694031) (end 128.461531 112.694031) (width 0.25) (layer "F.Cu") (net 3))
 (segment (start 131.025 88.398928) (end 131.025 88.845) (width 0.25) (layer "F.Cu") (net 7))
 (segment (start 128.175 109.212684) (end 128.175 110.17) (width 0.25) (layer "F.Cu") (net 7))
 (segment (start 132.703928 86.72) (end 131.025 88.398928) (width 0.25) (layer "F.Cu") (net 7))
 (segment (start 133.1125 109.545) (end 133.1625 109.595) (width 0.25) (layer "F.Cu") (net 7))
 (segment (start 133.546072 109.595) (end 134.175 110.223928) (width 0.25) (layer "F.Cu") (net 7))
 (segment (start 130.77452 110.64548) (end 130.9625 110.4575) (width 0.25) (layer "F.Cu") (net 7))
 (segment (start 127.732796 108.77048) (end 128.175 109.212684) (width 0.25) (layer "F.Cu") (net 7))
 (segment (start 130.9625 109.545) (end 133.1125 109.545) (width 0.25) (layer "F.Cu") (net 7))
 (segment (start 124.52548 108.77048) (end 127.732796 108.77048) (width 0.25) (layer "F.Cu") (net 7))
 (segment (start 133.335 86.72) (end 132.703928 86.72) (width 0.25) (layer "F.Cu") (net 7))
 (segment (start 130.9625 110.4575) (end 130.9625 111.4075) (width 0.25) (layer "F.Cu") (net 7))
 (segment (start 130.9625 111.4075) (end 130.925 111.445) (width 0.25) (layer "F.Cu") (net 7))
 (segment (start 130.9625 109.545) (end 130.9625 110.4575) (width 0.25) (layer "F.Cu") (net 7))
 (segment (start 123.150489 101.424511) (end 123.150489 107.395489) (width 0.25) (layer "F.Cu") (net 7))
 (segment (start 134.175 110.866072) (end 133.546072 111.495) (width 0.25) (layer "F.Cu") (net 7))
 (segment (start 133.546072 111.495) (end 133.1625 111.495) (width 0.25) (layer "F.Cu") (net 7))
 (segment (start 134.175 110.223928) (end 134.175 110.866072) (width 0.25) (layer "F.Cu") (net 7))
 (segment (start 128.175 110.17) (end 128.65048 110.64548) (width 0.25) (layer "F.Cu") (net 7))
 (segment (start 133.1625 109.595) (end 133.546072 109.595) (width 0.25) (layer "F.Cu") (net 7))
 (segment (start 124.075 100.5) (end 123.150489 101.424511) (width 0.25) (layer "F.Cu") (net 7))
 (segment (start 123.150489 107.395489) (end 124.52548 108.77048) (width 0.25) (layer "F.Cu") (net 7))
 (segment (start 128.65048 110.64548) (end 130.77452 110.64548) (width 0.25) (layer "F.Cu") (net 7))
 (segment (start 129.58002 90.47498) (end 125.073216 90.47498) (width 0.25) (layer "B.Cu") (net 7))
 (segment (start 133.335 86.72) (end 129.58002 90.47498) (width 0.25) (layer "B.Cu") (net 7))
 (segment (start 122.624511 92.923685) (end 122.624511 99.049511) (width 0.25) (layer "B.Cu") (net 7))
 (segment (start 122.624511 99.049511) (end 124.075 100.5) (width 0.25) (layer "B.Cu") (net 7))
 (segment (start 125.073216 90.47498) (end 122.624511 92.923685) (width 0.25) (layer "B.Cu") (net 7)))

